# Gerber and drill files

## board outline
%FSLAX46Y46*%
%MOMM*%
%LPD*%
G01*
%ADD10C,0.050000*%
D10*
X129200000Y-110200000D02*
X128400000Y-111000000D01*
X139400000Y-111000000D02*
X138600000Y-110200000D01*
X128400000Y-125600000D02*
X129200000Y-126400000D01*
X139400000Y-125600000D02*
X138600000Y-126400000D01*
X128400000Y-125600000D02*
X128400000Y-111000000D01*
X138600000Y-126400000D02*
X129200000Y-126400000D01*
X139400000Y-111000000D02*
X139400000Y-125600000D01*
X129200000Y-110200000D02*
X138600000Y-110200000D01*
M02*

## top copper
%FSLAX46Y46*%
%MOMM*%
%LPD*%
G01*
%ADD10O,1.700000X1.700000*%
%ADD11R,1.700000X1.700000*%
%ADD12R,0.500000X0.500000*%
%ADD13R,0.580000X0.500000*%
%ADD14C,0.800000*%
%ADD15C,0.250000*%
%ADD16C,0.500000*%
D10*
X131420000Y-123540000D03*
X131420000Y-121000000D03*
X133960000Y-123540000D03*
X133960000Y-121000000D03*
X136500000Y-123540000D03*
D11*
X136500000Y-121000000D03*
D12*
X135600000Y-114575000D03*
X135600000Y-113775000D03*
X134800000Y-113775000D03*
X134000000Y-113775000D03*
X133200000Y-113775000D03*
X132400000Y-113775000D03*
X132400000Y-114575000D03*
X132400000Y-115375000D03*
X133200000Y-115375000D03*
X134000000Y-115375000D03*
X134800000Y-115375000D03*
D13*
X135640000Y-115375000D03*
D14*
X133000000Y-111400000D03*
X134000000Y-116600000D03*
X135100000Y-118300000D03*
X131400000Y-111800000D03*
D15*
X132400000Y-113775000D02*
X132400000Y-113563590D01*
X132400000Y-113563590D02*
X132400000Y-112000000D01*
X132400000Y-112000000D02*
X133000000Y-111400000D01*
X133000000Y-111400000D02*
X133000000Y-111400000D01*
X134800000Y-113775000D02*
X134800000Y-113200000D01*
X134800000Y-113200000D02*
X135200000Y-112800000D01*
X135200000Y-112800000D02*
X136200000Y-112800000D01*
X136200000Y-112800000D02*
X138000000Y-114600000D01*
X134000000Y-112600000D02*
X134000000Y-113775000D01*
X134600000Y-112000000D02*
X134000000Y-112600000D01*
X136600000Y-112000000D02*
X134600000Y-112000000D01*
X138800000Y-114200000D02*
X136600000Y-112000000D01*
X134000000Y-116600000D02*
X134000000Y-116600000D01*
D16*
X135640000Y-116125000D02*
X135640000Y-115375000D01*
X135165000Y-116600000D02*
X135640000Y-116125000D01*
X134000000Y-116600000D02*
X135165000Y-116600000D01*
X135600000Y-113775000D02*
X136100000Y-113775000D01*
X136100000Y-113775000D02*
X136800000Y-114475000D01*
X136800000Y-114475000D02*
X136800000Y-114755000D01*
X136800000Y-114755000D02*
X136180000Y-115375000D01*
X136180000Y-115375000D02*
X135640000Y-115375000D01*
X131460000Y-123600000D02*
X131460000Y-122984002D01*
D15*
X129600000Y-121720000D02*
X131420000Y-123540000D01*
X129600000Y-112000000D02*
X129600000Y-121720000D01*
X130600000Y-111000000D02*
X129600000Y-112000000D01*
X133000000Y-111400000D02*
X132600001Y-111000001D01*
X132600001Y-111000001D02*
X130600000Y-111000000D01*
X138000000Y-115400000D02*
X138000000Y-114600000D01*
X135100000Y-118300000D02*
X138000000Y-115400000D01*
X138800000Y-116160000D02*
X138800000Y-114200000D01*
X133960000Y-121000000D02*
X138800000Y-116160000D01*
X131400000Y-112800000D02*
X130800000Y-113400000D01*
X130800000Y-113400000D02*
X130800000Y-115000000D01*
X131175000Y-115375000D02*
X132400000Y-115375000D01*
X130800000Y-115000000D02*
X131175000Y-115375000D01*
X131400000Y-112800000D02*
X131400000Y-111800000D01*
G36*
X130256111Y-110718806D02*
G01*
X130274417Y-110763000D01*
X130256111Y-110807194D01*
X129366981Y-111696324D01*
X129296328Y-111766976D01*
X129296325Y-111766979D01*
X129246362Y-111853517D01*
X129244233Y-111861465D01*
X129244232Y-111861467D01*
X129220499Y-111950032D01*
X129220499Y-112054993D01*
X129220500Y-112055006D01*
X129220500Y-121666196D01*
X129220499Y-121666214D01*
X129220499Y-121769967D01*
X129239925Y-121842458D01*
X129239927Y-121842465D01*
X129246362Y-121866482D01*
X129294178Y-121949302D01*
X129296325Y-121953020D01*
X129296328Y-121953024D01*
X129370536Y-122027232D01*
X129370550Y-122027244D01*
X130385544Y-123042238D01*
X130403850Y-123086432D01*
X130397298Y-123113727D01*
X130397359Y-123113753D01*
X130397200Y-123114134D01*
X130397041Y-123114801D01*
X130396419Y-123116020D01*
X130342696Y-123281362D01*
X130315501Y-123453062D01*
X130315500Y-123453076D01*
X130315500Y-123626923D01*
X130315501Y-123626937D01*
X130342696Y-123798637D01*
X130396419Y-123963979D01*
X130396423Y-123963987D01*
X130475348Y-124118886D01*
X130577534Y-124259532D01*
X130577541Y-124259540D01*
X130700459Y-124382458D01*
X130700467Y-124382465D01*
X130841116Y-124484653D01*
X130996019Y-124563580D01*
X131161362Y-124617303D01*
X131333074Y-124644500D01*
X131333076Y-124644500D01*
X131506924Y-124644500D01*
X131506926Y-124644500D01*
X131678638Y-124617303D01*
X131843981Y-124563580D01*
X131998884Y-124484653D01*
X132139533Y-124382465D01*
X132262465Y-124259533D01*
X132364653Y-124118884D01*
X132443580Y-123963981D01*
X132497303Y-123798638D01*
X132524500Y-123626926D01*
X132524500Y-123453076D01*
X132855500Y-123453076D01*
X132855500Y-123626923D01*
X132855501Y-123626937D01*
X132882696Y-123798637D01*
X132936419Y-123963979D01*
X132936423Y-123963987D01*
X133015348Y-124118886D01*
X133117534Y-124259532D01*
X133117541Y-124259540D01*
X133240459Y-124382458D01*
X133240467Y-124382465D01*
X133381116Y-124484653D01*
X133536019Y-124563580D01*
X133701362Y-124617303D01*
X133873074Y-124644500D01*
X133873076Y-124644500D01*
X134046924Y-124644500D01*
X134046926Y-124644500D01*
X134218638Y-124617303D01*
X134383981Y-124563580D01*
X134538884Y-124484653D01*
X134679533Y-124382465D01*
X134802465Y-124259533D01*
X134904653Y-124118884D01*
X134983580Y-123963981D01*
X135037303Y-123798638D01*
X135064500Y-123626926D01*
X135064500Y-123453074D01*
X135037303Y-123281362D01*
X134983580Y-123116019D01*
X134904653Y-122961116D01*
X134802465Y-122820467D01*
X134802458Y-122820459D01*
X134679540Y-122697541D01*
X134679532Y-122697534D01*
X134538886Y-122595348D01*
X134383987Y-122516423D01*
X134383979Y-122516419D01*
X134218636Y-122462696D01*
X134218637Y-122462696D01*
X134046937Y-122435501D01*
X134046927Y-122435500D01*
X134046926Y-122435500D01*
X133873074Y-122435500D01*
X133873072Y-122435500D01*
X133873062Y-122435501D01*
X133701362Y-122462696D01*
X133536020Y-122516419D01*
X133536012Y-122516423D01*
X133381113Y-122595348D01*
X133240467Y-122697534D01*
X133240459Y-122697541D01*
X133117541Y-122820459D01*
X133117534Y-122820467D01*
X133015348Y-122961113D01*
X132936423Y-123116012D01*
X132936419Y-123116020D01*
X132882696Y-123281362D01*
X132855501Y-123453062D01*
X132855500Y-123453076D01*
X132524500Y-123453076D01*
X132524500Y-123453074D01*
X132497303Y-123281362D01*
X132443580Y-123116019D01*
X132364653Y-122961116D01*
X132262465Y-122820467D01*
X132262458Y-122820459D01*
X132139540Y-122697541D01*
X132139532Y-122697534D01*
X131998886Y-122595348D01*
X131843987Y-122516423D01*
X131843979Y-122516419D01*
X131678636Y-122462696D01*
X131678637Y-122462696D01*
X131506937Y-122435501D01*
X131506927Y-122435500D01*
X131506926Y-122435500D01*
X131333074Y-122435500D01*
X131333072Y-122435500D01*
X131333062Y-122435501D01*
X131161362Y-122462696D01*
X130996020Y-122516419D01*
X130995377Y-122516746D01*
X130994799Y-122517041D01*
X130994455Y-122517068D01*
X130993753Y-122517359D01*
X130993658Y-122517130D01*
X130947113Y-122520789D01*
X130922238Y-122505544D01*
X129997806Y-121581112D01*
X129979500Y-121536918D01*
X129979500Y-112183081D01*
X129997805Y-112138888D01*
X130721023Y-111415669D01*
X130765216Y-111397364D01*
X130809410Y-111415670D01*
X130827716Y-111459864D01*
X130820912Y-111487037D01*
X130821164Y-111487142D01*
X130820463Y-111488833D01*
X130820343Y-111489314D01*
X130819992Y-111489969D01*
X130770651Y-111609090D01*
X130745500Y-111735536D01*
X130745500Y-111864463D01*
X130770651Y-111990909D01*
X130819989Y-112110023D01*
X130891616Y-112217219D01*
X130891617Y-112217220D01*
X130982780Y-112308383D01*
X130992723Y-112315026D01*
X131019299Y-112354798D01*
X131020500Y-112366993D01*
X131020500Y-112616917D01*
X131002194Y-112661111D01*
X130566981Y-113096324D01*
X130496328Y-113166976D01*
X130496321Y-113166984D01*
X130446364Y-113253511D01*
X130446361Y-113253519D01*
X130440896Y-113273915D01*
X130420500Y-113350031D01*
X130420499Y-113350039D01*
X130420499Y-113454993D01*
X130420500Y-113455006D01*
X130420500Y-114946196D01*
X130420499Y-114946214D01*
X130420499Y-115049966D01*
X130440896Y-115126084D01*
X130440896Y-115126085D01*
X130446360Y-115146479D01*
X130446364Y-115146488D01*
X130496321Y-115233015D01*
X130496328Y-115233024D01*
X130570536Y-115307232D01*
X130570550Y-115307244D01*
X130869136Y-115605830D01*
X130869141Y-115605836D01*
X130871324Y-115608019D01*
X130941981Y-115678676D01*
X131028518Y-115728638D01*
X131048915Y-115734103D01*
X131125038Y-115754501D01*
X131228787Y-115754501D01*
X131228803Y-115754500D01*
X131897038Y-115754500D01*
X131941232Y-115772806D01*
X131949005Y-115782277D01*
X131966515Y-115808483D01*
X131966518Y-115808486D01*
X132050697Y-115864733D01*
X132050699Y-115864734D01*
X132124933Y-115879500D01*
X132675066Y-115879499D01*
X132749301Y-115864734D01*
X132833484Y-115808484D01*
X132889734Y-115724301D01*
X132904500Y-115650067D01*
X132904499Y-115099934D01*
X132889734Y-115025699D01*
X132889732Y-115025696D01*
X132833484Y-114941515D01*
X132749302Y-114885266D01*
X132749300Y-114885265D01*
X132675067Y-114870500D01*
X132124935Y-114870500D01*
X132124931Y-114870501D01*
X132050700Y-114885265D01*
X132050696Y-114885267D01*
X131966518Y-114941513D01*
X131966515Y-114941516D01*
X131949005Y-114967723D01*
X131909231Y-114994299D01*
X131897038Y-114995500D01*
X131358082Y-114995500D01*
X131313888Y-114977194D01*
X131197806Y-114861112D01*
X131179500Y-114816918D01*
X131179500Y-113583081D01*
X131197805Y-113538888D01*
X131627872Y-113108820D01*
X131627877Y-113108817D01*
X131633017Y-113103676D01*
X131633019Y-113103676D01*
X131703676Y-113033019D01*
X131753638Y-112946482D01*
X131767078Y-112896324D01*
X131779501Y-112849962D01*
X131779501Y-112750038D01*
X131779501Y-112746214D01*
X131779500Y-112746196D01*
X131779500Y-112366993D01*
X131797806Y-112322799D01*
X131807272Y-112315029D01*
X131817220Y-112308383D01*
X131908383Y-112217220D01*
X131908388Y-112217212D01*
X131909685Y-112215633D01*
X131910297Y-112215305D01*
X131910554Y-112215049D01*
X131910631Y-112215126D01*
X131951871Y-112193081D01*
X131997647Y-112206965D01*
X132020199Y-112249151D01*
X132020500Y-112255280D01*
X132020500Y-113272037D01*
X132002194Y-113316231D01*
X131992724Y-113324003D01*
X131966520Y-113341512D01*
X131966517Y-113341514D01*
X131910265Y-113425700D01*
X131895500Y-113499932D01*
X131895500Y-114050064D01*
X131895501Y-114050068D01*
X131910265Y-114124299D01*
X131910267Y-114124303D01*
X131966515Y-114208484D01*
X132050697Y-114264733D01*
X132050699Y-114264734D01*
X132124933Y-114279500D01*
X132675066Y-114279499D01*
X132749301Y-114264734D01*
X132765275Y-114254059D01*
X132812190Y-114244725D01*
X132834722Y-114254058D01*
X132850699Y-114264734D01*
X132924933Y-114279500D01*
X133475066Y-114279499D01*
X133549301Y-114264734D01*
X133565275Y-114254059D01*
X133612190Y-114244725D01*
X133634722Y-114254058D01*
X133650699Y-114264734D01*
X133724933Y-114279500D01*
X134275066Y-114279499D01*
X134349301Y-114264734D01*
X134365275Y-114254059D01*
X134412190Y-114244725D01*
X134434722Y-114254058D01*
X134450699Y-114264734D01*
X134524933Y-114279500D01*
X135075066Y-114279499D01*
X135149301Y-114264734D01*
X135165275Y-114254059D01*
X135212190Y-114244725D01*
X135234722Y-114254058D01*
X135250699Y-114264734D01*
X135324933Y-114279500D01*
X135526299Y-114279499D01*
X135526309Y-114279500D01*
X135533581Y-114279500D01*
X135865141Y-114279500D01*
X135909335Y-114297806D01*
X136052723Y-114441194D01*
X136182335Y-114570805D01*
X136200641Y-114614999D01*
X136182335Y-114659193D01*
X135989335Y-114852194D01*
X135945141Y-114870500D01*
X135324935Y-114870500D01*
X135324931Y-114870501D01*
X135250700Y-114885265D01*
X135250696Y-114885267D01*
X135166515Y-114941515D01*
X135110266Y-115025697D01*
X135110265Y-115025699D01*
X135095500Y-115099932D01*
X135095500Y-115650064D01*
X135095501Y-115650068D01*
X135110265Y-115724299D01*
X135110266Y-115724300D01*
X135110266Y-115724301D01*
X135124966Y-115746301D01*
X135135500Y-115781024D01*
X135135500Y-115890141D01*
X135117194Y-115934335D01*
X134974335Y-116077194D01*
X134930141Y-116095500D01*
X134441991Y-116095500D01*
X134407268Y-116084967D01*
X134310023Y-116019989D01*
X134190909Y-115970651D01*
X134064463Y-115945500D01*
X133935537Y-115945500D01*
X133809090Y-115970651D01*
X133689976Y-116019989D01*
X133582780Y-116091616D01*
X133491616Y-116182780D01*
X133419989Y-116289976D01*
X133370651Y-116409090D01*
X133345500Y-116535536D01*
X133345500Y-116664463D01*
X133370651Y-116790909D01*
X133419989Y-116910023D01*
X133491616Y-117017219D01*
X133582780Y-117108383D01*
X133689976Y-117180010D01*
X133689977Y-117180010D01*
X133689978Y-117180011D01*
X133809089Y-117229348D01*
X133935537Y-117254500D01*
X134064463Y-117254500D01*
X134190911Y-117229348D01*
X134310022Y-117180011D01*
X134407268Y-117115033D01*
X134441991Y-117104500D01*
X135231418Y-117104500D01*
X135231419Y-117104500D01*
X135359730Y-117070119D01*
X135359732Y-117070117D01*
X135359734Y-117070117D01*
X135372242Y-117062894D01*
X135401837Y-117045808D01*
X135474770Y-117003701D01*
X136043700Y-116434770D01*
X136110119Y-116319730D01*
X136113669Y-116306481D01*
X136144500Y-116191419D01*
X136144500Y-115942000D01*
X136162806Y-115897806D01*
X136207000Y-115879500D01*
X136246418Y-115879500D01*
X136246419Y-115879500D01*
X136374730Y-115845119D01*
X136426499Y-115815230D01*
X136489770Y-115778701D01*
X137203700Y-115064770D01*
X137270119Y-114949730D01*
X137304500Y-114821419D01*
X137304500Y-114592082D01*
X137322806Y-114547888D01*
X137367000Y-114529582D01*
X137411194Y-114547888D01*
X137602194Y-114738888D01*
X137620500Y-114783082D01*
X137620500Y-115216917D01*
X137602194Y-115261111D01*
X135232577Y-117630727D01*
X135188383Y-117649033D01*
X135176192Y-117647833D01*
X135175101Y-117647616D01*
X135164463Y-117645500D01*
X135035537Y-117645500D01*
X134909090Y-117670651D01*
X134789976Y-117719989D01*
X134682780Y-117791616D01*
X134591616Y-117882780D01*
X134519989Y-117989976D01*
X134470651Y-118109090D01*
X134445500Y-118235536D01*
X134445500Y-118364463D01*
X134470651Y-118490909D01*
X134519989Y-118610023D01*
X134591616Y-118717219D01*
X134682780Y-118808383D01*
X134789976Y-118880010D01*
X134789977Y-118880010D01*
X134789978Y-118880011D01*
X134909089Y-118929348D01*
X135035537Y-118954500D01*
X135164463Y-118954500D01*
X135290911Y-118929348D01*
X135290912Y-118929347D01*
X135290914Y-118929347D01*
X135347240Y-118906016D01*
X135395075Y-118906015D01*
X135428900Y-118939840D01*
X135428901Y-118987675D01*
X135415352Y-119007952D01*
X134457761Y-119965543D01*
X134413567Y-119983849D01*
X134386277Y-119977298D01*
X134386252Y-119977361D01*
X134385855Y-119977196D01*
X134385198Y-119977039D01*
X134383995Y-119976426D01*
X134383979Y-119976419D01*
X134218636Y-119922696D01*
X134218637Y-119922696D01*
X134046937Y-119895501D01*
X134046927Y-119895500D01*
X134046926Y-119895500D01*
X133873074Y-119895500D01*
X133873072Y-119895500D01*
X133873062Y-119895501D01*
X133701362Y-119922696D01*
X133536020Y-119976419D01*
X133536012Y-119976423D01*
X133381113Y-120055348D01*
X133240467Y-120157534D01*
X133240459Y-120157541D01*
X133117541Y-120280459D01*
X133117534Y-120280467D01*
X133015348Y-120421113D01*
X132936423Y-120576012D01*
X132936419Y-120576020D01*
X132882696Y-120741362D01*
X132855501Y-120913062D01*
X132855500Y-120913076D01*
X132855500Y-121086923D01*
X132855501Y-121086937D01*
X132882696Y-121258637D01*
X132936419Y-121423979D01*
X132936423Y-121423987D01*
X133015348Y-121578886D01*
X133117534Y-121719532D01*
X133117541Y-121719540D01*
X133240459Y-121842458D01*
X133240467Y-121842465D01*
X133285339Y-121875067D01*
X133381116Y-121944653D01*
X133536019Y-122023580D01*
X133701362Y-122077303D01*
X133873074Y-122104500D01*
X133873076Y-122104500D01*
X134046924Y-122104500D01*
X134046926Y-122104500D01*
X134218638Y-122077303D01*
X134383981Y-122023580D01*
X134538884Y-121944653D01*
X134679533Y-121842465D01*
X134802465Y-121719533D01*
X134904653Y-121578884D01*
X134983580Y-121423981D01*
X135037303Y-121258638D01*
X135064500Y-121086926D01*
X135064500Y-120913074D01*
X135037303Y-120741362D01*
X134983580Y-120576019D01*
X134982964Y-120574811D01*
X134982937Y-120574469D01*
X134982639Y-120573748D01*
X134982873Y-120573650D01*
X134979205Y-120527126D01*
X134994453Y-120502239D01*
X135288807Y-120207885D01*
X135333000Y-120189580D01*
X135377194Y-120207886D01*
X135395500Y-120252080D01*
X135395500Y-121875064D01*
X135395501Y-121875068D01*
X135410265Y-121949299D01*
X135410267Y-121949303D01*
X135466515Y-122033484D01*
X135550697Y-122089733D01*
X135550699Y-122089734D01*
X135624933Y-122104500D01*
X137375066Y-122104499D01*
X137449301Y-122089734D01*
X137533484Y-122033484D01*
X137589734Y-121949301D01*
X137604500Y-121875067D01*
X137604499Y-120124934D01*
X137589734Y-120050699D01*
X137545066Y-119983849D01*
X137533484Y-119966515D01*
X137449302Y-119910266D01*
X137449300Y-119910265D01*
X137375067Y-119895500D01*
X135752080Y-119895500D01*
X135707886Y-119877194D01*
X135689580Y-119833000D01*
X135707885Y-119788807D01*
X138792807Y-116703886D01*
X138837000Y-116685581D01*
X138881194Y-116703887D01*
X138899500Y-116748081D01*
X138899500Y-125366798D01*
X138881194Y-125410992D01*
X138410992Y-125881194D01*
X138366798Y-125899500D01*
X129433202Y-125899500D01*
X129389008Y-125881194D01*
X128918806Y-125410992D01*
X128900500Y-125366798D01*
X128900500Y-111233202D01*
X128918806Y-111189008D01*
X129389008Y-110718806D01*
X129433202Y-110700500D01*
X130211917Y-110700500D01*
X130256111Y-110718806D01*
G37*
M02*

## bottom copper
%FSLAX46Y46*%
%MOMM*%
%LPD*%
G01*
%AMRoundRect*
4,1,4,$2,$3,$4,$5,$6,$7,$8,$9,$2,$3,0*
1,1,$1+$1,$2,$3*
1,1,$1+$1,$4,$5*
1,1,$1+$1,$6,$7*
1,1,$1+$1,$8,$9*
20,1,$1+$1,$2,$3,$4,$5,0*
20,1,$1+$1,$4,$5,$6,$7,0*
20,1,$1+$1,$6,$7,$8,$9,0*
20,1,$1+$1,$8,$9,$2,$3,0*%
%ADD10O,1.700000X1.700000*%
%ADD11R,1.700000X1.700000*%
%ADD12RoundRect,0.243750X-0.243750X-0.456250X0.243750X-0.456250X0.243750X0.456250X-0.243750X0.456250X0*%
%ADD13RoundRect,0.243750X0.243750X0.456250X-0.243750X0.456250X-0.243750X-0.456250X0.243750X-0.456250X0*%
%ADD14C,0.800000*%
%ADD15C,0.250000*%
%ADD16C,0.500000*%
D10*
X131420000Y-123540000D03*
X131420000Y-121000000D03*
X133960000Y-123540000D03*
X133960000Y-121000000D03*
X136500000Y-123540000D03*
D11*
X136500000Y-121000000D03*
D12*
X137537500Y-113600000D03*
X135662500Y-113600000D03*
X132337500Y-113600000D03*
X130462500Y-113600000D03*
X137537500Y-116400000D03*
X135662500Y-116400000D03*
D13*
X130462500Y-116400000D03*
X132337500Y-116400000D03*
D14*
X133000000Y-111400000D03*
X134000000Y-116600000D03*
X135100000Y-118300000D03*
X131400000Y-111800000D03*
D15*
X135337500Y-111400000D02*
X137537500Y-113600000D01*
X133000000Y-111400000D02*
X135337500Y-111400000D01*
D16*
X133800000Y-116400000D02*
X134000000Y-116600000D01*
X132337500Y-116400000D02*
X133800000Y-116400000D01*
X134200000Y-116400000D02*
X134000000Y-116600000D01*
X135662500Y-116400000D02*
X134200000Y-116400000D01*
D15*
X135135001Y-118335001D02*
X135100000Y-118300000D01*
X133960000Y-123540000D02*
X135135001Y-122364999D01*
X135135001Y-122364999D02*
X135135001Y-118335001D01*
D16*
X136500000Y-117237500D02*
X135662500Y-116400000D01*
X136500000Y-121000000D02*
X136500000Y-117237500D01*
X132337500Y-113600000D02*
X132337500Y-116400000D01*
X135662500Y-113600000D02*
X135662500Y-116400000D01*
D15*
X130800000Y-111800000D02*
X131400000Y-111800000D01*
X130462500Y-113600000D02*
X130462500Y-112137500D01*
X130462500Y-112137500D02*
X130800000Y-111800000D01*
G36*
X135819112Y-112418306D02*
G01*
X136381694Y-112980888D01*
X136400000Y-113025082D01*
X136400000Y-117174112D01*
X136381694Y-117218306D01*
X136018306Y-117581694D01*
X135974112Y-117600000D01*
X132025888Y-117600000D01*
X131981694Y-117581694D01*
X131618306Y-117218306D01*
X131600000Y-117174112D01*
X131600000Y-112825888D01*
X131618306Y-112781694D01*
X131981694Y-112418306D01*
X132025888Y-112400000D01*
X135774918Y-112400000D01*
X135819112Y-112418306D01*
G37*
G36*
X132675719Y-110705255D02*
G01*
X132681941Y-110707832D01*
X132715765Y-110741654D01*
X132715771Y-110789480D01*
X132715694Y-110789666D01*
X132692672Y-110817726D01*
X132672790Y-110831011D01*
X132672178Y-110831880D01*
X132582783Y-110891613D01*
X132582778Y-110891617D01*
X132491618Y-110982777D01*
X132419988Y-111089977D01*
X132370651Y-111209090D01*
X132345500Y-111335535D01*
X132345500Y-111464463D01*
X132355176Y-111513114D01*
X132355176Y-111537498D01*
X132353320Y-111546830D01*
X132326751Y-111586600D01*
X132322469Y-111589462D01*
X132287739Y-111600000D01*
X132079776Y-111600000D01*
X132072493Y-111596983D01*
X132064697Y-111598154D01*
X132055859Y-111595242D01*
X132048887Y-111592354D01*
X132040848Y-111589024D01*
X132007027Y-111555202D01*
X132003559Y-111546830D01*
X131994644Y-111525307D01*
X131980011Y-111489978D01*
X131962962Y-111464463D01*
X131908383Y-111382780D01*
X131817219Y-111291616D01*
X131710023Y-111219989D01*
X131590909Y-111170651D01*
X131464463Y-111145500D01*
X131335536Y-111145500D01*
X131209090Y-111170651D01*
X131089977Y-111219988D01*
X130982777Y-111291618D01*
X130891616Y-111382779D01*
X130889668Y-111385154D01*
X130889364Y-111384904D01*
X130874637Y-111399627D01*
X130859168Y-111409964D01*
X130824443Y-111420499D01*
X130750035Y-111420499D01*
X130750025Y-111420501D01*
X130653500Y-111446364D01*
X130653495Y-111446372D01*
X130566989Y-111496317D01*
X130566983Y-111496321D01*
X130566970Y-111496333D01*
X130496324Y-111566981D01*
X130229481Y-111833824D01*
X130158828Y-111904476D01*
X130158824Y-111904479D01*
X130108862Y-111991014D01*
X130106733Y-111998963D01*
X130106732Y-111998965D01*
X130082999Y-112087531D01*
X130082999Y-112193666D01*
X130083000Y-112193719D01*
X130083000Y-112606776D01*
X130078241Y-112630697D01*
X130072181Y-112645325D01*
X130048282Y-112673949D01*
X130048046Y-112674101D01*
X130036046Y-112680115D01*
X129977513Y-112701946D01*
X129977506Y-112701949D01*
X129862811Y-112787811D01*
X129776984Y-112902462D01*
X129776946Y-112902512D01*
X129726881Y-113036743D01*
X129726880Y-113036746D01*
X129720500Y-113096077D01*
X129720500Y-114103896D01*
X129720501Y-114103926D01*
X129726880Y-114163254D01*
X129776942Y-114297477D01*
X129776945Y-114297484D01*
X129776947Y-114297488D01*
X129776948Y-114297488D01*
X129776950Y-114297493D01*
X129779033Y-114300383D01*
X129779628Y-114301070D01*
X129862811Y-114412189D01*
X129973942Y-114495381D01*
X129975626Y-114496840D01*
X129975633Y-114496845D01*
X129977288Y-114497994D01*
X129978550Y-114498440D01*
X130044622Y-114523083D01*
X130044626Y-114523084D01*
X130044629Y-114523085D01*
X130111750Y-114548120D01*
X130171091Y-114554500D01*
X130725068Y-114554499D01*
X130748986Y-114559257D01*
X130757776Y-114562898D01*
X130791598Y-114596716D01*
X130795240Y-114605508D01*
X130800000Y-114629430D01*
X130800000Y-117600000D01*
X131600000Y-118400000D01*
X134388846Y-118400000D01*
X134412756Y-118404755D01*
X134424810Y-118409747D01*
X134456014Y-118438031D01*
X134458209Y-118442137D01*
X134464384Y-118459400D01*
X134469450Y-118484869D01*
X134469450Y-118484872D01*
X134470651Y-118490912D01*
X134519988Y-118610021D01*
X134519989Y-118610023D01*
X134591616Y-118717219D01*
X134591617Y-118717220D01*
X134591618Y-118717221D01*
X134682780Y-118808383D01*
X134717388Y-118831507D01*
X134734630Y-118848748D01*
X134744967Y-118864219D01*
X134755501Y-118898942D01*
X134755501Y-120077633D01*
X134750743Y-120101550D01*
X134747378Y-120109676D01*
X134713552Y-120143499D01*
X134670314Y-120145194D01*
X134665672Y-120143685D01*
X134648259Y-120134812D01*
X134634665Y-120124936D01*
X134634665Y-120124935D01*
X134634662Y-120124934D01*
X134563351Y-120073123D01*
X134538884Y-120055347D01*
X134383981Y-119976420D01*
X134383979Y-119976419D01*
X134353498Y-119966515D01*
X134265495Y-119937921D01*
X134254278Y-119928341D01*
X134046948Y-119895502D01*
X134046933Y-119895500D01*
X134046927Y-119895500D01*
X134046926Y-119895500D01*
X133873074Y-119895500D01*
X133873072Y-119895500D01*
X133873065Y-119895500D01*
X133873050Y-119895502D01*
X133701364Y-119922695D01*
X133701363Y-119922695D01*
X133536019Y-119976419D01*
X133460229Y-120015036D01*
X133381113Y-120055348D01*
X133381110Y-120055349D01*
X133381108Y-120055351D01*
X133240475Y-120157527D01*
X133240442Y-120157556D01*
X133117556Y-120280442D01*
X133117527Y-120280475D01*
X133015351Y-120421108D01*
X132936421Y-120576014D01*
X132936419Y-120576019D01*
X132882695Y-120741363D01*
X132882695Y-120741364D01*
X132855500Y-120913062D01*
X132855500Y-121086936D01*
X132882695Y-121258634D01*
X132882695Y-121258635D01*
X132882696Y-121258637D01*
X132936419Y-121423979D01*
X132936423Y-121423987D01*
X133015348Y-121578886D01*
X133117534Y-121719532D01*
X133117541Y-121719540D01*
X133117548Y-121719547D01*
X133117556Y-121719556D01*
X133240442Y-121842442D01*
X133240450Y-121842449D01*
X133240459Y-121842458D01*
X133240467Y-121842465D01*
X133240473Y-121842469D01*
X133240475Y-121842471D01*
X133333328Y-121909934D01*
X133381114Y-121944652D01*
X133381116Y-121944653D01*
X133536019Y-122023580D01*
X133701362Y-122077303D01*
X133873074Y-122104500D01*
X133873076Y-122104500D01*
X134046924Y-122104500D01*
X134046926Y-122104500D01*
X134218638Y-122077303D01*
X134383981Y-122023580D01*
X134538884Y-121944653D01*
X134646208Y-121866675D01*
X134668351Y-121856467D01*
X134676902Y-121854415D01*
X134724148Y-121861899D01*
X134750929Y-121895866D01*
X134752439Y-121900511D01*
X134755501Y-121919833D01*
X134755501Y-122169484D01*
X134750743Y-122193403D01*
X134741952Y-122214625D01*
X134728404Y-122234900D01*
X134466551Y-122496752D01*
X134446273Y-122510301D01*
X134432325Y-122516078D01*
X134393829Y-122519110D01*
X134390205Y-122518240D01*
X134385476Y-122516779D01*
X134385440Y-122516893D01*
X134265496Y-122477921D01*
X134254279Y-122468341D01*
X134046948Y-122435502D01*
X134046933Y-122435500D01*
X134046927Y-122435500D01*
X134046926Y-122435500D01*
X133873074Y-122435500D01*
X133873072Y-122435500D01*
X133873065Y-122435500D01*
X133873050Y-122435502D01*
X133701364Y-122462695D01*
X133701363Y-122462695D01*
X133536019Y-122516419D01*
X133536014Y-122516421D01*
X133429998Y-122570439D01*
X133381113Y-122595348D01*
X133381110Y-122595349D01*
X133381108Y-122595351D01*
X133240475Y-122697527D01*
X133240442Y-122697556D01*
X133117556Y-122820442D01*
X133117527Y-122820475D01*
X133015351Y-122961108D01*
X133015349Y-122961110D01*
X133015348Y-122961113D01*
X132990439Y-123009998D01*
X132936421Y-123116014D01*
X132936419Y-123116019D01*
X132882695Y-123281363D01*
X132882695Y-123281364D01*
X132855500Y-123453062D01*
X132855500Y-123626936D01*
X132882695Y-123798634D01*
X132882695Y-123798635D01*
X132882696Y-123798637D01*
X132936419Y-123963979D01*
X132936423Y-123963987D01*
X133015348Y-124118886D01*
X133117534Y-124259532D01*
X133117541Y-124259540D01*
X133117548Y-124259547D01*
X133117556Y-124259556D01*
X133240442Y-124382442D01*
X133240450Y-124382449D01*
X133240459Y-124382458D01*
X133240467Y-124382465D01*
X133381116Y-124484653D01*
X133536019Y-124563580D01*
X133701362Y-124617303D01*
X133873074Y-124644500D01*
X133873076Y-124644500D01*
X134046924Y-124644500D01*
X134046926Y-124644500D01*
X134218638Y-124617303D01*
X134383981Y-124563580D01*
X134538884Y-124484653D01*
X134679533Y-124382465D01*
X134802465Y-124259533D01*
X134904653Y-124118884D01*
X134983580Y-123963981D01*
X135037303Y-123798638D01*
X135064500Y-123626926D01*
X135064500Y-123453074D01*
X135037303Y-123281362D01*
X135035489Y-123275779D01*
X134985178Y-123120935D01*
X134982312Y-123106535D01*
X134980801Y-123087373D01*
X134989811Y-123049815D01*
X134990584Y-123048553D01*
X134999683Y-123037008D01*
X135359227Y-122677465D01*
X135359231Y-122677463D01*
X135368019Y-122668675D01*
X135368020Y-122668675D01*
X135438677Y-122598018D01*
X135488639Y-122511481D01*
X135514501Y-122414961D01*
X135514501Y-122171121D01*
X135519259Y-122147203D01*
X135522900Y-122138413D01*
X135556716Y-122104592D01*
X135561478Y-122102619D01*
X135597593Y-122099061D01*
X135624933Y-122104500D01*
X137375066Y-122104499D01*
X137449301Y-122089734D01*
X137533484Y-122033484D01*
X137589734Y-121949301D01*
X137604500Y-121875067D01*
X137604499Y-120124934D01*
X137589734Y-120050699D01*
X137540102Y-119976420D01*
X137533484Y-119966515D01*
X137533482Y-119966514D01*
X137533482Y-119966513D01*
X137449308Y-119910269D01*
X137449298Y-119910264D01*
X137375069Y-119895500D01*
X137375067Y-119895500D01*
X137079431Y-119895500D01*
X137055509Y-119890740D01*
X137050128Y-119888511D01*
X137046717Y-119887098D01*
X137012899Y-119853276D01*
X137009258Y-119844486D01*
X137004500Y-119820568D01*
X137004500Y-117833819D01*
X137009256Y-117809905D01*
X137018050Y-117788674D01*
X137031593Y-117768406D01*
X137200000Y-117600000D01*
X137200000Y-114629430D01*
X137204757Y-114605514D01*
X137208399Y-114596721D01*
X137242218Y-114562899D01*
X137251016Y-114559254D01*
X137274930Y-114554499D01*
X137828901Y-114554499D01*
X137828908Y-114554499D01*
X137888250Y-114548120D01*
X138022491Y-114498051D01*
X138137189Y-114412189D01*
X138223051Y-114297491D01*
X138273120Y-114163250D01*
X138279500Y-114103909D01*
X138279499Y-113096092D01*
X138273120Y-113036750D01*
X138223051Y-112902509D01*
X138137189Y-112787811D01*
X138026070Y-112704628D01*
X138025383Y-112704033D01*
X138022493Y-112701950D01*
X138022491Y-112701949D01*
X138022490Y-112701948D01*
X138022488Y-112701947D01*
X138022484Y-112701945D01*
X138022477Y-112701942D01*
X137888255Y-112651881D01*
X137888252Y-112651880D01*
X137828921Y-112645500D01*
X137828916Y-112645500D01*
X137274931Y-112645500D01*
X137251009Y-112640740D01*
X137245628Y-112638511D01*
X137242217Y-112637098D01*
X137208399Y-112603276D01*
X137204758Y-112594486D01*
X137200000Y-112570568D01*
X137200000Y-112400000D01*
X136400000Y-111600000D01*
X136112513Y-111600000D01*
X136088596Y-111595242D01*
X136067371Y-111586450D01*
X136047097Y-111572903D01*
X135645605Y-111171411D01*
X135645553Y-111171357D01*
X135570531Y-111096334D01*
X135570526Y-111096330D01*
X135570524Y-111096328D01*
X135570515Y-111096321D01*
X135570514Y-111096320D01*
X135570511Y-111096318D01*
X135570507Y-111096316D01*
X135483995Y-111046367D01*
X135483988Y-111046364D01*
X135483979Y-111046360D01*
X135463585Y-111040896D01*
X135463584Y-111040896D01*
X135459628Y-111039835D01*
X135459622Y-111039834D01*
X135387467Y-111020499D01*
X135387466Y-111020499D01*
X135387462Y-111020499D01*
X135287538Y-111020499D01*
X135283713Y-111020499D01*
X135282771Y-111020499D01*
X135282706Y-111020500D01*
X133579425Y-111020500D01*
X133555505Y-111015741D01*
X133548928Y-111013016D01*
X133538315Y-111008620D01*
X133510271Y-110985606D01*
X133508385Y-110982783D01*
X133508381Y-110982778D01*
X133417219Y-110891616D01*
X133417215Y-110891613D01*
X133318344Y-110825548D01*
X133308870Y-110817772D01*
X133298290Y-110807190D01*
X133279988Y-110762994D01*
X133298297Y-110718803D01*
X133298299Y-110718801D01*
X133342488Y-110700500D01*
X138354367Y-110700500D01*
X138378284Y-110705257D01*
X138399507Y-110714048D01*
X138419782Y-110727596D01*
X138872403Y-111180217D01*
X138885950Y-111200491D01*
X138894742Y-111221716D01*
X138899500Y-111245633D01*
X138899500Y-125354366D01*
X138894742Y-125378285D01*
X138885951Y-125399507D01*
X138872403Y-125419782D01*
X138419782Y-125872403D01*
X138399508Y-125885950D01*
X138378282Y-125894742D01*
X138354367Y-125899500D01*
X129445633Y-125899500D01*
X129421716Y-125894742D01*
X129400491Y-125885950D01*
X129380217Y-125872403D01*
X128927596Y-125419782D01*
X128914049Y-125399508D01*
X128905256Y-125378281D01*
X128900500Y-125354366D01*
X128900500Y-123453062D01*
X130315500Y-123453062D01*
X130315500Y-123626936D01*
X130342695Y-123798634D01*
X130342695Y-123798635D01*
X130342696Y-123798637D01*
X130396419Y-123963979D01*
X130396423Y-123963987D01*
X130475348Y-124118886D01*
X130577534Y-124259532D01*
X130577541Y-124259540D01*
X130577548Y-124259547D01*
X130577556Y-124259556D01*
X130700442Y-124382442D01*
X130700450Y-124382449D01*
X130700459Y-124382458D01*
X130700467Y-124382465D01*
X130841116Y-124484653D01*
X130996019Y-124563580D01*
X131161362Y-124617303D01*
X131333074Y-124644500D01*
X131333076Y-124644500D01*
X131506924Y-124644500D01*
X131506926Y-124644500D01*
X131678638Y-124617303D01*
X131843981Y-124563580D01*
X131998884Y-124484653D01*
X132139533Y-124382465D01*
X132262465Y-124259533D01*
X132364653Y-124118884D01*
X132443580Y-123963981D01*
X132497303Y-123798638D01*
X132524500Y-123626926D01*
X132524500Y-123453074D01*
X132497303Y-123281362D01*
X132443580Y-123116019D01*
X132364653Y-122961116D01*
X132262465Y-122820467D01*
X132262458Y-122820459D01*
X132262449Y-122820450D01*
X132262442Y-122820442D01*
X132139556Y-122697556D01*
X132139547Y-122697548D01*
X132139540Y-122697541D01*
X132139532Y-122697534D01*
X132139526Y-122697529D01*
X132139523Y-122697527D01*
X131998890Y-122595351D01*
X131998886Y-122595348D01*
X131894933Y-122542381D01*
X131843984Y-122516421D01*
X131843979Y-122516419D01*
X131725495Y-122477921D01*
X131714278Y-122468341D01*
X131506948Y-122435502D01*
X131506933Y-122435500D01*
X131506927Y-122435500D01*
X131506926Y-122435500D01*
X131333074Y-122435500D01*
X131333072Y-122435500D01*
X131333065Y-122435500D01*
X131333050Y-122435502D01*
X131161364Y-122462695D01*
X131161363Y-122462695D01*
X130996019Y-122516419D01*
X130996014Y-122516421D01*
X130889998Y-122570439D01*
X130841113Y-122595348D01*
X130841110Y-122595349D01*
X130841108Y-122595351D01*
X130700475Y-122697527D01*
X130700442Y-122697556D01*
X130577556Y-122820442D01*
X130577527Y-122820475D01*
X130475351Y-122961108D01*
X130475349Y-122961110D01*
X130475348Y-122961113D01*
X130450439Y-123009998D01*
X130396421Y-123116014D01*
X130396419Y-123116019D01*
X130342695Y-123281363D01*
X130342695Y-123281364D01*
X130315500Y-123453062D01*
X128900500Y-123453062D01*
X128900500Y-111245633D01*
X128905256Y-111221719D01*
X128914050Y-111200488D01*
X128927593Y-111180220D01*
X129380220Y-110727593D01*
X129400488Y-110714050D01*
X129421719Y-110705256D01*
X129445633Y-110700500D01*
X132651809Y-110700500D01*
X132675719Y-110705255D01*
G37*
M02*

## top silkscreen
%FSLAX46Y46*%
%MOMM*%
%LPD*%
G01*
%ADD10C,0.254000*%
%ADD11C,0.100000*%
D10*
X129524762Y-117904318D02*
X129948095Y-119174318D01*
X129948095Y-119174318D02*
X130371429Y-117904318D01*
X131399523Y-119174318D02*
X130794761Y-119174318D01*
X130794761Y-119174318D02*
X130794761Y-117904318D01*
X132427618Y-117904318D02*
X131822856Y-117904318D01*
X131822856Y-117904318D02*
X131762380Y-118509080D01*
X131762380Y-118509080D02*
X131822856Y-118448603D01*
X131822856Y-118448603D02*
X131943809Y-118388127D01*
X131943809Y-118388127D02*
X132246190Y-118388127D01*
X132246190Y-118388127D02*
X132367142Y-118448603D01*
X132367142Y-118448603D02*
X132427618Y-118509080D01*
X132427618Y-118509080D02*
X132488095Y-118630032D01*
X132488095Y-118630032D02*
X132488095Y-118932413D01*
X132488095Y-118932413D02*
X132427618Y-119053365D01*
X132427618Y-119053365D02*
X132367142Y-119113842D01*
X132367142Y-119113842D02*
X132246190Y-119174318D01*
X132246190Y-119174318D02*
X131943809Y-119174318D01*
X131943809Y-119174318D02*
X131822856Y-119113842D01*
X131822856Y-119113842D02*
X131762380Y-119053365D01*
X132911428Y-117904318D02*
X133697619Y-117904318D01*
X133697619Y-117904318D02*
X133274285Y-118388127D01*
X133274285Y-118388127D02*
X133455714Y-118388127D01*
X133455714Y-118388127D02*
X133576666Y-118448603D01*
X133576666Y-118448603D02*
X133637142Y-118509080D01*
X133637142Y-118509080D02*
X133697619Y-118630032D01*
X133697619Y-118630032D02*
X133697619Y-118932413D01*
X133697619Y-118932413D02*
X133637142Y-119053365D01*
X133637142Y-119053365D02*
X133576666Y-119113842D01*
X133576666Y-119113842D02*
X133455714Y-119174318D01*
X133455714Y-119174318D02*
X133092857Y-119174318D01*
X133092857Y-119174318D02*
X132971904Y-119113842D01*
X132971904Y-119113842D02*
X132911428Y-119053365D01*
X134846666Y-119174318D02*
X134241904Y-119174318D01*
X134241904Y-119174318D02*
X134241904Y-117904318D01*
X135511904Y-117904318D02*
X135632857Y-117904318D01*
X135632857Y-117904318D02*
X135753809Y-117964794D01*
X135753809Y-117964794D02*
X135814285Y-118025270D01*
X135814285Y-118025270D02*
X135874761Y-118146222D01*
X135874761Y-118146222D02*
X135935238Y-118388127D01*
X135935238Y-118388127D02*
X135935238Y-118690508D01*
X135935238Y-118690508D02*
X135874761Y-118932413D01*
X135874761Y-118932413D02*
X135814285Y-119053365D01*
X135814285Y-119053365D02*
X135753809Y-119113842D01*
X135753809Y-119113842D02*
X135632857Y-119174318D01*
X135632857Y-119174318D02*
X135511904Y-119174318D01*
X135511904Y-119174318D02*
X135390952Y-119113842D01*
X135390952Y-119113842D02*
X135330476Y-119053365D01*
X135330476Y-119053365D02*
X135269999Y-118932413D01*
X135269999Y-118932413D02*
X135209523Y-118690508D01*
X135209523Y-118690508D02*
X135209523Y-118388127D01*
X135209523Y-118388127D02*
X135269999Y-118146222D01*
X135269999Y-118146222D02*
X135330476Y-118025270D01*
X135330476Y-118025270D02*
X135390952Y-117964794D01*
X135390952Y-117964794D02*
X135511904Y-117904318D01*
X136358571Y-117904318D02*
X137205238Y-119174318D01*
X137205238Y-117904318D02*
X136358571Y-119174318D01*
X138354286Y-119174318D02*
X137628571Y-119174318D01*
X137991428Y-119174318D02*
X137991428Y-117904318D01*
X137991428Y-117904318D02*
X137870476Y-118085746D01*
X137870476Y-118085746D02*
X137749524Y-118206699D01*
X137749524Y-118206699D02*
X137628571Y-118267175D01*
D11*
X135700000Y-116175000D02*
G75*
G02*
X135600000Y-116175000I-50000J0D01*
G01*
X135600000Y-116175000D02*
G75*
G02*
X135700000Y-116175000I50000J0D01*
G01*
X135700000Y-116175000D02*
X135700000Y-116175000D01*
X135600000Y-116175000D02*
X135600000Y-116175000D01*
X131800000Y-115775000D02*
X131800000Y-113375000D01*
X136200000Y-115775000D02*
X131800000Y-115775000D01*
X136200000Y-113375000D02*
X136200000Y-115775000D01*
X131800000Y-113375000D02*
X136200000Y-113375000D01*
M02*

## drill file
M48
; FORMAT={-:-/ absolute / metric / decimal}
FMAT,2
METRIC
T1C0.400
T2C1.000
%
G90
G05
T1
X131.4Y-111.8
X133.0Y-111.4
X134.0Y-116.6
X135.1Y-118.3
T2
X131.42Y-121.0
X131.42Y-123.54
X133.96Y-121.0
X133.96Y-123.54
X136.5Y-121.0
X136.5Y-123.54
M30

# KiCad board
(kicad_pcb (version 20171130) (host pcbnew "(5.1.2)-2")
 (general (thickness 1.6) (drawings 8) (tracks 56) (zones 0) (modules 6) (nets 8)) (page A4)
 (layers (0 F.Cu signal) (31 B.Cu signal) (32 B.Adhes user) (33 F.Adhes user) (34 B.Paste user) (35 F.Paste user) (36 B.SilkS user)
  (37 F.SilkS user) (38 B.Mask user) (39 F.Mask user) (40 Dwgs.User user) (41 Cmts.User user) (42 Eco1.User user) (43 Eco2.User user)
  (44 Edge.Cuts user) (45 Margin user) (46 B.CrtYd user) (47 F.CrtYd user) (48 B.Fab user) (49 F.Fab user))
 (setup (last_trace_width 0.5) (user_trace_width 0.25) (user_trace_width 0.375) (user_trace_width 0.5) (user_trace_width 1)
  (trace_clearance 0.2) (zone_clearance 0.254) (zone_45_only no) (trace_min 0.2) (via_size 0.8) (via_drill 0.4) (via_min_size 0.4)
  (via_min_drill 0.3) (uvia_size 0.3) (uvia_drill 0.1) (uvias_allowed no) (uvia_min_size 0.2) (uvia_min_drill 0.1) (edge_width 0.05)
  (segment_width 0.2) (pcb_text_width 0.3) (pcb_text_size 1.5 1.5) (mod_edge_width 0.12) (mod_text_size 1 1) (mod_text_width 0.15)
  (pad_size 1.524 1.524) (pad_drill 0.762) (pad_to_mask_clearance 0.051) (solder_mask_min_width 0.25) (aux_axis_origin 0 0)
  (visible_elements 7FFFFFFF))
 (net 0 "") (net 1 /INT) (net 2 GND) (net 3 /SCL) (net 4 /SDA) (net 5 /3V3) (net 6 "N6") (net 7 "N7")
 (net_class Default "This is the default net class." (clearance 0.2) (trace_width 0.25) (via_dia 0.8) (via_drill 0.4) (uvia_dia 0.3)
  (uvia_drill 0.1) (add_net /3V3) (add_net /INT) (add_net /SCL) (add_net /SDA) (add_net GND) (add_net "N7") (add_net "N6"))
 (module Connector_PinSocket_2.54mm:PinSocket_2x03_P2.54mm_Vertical (layer B.Cu) (at 136.5 121 90)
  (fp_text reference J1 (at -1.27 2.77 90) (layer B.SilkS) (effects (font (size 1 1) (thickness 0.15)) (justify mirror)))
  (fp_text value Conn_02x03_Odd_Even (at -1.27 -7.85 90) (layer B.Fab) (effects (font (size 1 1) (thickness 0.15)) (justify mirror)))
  (pad 6 thru_hole oval (at -2.54 -5.08 90) (size 1.7 1.7) (drill 1) (layers *.Cu *.Mask) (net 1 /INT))
  (pad 5 thru_hole oval (at 0 -5.08 90) (size 1.7 1.7) (drill 1) (layers *.Cu *.Mask) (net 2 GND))
  (pad 4 thru_hole oval (at -2.54 -2.54 90) (size 1.7 1.7) (drill 1) (layers *.Cu *.Mask) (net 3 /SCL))
  (pad 3 thru_hole oval (at 0 -2.54 90) (size 1.7 1.7) (drill 1) (layers *.Cu *.Mask) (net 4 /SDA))
  (pad 2 thru_hole oval (at -2.54 0 90) (size 1.7 1.7) (drill 1) (layers *.Cu *.Mask) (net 2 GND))
  (pad 1 thru_hole rect (at 0 0 90) (size 1.7 1.7) (drill 1) (layers *.Cu *.Mask) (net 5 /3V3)))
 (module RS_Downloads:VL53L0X (layer F.Cu) (at 134 114.8)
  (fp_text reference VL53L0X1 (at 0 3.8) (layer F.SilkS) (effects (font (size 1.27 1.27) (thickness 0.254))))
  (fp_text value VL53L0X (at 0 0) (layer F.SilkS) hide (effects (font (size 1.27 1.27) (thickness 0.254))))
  (fp_arc (start 1.65 1.375) (end 1.7 1.375) (angle 180) (layer F.SilkS) (width 0.1))
  (fp_arc (start 1.65 1.375) (end 1.6 1.375) (angle 180) (layer F.SilkS) (width 0.1))
  (fp_line (start 1.7 1.375) (end 1.7 1.375) (layer F.SilkS) (width 0.1))
  (fp_line (start 1.6 1.375) (end 1.6 1.375) (layer F.SilkS) (width 0.1))
  (fp_line (start -2.2 0.975) (end -2.2 -1.425) (layer F.SilkS) (width 0.1))
  (fp_line (start 2.2 0.975) (end -2.2 0.975) (layer F.SilkS) (width 0.1))
  (fp_line (start 2.2 -1.425) (end 2.2 0.975) (layer F.SilkS) (width 0.1))
  (fp_line (start -2.2 -1.425) (end 2.2 -1.425) (layer F.SilkS) (width 0.1))
  (pad 12 smd rect (at 1.6 -0.225 90) (size 0.5 0.5) (layers F.Cu F.Paste F.Mask) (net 2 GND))
  (pad 11 smd rect (at 1.6 -1.025 90) (size 0.5 0.5) (layers F.Cu F.Paste F.Mask) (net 5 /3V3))
  (pad 10 smd rect (at 0.8 -1.025 90) (size 0.5 0.5) (layers F.Cu F.Paste F.Mask) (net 3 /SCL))
  (pad 9 smd rect (at 0 -1.025 90) (size 0.5 0.5) (layers F.Cu F.Paste F.Mask) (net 4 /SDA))
  (pad 8 smd rect (at -0.8 -1.025 90) (size 0.5 0.5) (layers F.Cu F.Paste F.Mask) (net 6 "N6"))
  (pad 7 smd rect (at -1.6 -1.025 90) (size 0.5 0.5) (layers F.Cu F.Paste F.Mask) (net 1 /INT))
  (pad 6 smd rect (at -1.6 -0.225 90) (size 0.5 0.5) (layers F.Cu F.Paste F.Mask) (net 2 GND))
  (pad 5 smd rect (at -1.6 0.575 90) (size 0.5 0.5) (layers F.Cu F.Paste F.Mask) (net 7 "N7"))
  (pad 4 smd rect (at -0.8 0.575 90) (size 0.5 0.5) (layers F.Cu F.Paste F.Mask) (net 2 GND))
  (pad 3 smd rect (at 0 0.575 90) (size 0.5 0.5) (layers F.Cu F.Paste F.Mask) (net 2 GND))
  (pad 2 smd rect (at 0.8 0.575 90) (size 0.5 0.5) (layers F.Cu F.Paste F.Mask) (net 2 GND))
  (pad 1 smd rect (at 1.64 0.575 90) (size 0.5 0.58) (layers F.Cu F.Paste F.Mask) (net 5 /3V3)))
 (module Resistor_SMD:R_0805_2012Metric (layer B.Cu) (at 136.6 113.6)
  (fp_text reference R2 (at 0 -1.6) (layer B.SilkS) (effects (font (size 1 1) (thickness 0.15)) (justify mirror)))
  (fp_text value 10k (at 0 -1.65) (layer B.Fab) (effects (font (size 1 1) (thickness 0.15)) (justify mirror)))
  (pad 2 smd roundrect (at 0.9375 0) (size 0.975 1.4) (layers B.Cu B.Paste B.Mask) (roundrect_rratio 0.25) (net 1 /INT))
  (pad 1 smd roundrect (at -0.9375 0) (size 0.975 1.4) (layers B.Cu B.Paste B.Mask) (roundrect_rratio 0.25) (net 5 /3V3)))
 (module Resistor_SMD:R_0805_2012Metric (layer B.Cu) (at 131.4 113.6)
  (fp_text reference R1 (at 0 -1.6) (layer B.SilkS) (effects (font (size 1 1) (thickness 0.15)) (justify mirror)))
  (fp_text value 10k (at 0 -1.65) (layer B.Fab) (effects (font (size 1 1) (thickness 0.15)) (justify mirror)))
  (pad 2 smd roundrect (at 0.9375 0) (size 0.975 1.4) (layers B.Cu B.Paste B.Mask) (roundrect_rratio 0.25) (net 5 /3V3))
  (pad 1 smd roundrect (at -0.9375 0) (size 0.975 1.4) (layers B.Cu B.Paste B.Mask) (roundrect_rratio 0.25) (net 7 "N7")))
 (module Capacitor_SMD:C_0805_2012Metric (layer B.Cu) (at 136.6 116.4)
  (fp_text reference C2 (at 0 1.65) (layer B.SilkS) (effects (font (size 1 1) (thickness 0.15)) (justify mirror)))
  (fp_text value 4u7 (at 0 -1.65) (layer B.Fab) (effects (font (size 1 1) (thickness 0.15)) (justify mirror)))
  (pad 2 smd roundrect (at 0.9375 0) (size 0.975 1.4) (layers B.Cu B.Paste B.Mask) (roundrect_rratio 0.25) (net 2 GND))
  (pad 1 smd roundrect (at -0.9375 0) (size 0.975 1.4) (layers B.Cu B.Paste B.Mask) (roundrect_rratio 0.25) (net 5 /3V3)))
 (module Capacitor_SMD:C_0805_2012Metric (layer B.Cu) (at 131.4 116.4 180)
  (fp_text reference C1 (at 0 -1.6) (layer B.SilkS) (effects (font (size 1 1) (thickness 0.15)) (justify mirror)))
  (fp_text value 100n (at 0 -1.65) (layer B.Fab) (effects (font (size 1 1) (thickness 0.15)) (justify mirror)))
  (pad 2 smd roundrect (at 0.9375 0 180) (size 0.975 1.4) (layers B.Cu B.Paste B.Mask) (roundrect_rratio 0.25) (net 2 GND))
  (pad 1 smd roundrect (at -0.9375 0 180) (size 0.975 1.4) (layers B.Cu B.Paste B.Mask) (roundrect_rratio 0.25) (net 5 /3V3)))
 (gr_line (start 129.2 110.2) (end 128.4 111) (layer Edge.Cuts) (width 0.05))
 (gr_line (start 139.4 111) (end 138.6 110.2) (layer Edge.Cuts) (width 0.05))
 (gr_line (start 128.4 125.6) (end 129.2 126.4) (layer Edge.Cuts) (width 0.05))
 (gr_line (start 139.4 125.6) (end 138.6 126.4) (layer Edge.Cuts) (width 0.05))
 (gr_line (start 128.4 125.6) (end 128.4 111) (layer Edge.Cuts) (width 0.05))
 (gr_line (start 138.6 126.4) (end 129.2 126.4) (layer Edge.Cuts) (width 0.05))
 (gr_line (start 139.4 111) (end 139.4 125.6) (layer Edge.Cuts) (width 0.05))
 (gr_line (start 129.2 110.2) (end 138.6 110.2) (layer Edge.Cuts) (width 0.05))
 (segment (start 132.4 113.775) (end 132.4 113.56359) (width 0.25) (layer F.Cu) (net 1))
 (segment (start 132.4 113.56359) (end 132.4 112) (width 0.25) (layer F.Cu) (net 1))
 (segment (start 132.4 112) (end 133 111.4) (width 0.25) (layer F.Cu) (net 1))
 (segment (start 133 111.4) (end 133 111.4) (width 0.25) (layer F.Cu) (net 1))
 (via (at 133 111.4) (size 0.8) (drill 0.4) (layers F.Cu B.Cu) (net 1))
 (segment (start 135.3375 111.4) (end 137.5375 113.6) (width 0.25) (layer B.Cu) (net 1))
 (segment (start 133 111.4) (end 135.3375 111.4) (width 0.25) (layer B.Cu) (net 1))
 (segment (start 134.8 113.775) (end 134.8 113.2) (width 0.25) (layer F.Cu) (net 3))
 (segment (start 134.8 113.2) (end 135.2 112.8) (width 0.25) (layer F.Cu) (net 3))
 (segment (start 135.2 112.8) (end 136.2 112.8) (width 0.25) (layer F.Cu) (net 3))
 (segment (start 136.2 112.8) (end 138 114.6) (width 0.25) (layer F.Cu) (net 3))
 (segment (start 134 112.6) (end 134 113.775) (width 0.25) (layer F.Cu) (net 4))
 (segment (start 134.6 112) (end 134 112.6) (width 0.25) (layer F.Cu) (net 4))
 (segment (start 136.6 112) (end 134.6 112) (width 0.25) (layer F.Cu) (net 4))
 (segment (start 138.8 114.2) (end 136.6 112) (width 0.25) (layer F.Cu) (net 4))
 (segment (start 134 116.6) (end 134 116.6) (width 0.25) (layer F.Cu) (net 5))
 (via (at 134 116.6) (size 0.8) (drill 0.4) (layers F.Cu B.Cu) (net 5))
 (segment (start 135.64 116.125) (end 135.64 115.375) (width 0.5) (layer F.Cu) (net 5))
 (segment (start 135.165 116.6) (end 135.64 116.125) (width 0.5) (layer F.Cu) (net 5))
 (segment (start 134 116.6) (end 135.165 116.6) (width 0.5) (layer F.Cu) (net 5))
 (segment (start 135.6 113.775) (end 136.1 113.775) (width 0.5) (layer F.Cu) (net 5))
 (segment (start 136.1 113.775) (end 136.8 114.475) (width 0.5) (layer F.Cu) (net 5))
 (segment (start 136.8 114.475) (end 136.8 114.755) (width 0.5) (layer F.Cu) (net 5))
 (segment (start 136.8 114.755) (end 136.18 115.375) (width 0.5) (layer F.Cu) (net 5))
 (segment (start 136.18 115.375) (end 135.64 115.375) (width 0.5) (layer F.Cu) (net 5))
 (segment (start 133.8 116.4) (end 134 116.6) (width 0.5) (layer B.Cu) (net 5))
 (segment (start 132.3375 116.4) (end 133.8 116.4) (width 0.5) (layer B.Cu) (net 5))
 (segment (start 134.2 116.4) (end 134 116.6) (width 0.5) (layer B.Cu) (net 5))
 (segment (start 135.6625 116.4) (end 134.2 116.4) (width 0.5) (layer B.Cu) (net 5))
 (segment (start 131.46 123.6) (end 131.46 122.984002) (width 0.5) (layer F.Cu) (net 1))
 (segment (start 129.6 121.72) (end 131.42 123.54) (width 0.25) (layer F.Cu) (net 1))
 (segment (start 129.6 112) (end 129.6 121.72) (width 0.25) (layer F.Cu) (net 1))
 (segment (start 130.6 111) (end 129.6 112) (width 0.25) (layer F.Cu) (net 1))
 (segment (start 133 111.4) (end 132.600001 111.000001) (width 0.25) (layer F.Cu) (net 1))
 (segment (start 132.600001 111.000001) (end 130.6 111) (width 0.25) (layer F.Cu) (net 1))
 (via (at 135.1 118.3) (size 0.8) (drill 0.4) (layers F.Cu B.Cu) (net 3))
 (segment (start 135.135001 118.335001) (end 135.1 118.3) (width 0.25) (layer B.Cu) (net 3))
 (segment (start 133.96 123.54) (end 135.135001 122.364999) (width 0.25) (layer B.Cu) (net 3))
 (segment (start 135.135001 122.364999) (end 135.135001 118.335001) (width 0.25) (layer B.Cu) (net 3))
 (segment (start 138 115.4) (end 138 114.6) (width 0.25) (layer F.Cu) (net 3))
 (segment (start 135.1 118.3) (end 138 115.4) (width 0.25) (layer F.Cu) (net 3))
 (segment (start 138.8 116.16) (end 138.8 114.2) (width 0.25) (layer F.Cu) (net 4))
 (segment (start 133.96 121) (end 138.8 116.16) (width 0.25) (layer F.Cu) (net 4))
 (segment (start 136.5 117.2375) (end 135.6625 116.4) (width 0.5) (layer B.Cu) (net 5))
 (segment (start 136.5 121) (end 136.5 117.2375) (width 0.5) (layer B.Cu) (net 5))
 (segment (start 132.3375 113.6) (end 132.3375 116.4) (width 0.5) (layer B.Cu) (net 5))
 (segment (start 135.6625 113.6) (end 135.6625 116.4) (width 0.5) (layer B.Cu) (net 5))
 (via (at 131.4 111.8) (size 0.8) (drill 0.4) (layers F.Cu B.Cu) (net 7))
 (segment (start 131.4 112.8) (end 130.8 113.4) (width 0.25) (layer F.Cu) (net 7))
 (segment (start 130.8 113.4) (end 130.8 115) (width 0.25) (layer F.Cu) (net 7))
 (segment (start 131.175 115.375) (end 132.4 115.375) (width 0.25) (layer F.Cu) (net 7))
 (segment (start 130.8 115) (end 131.175 115.375) (width 0.25) (layer F.Cu) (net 7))
 (segment (start 131.4 112.8) (end 131.4 111.8) (width 0.25) (layer F.Cu) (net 7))
 (segment (start 130.8 111.8) (end 131.4 111.8) (width 0.25) (layer B.Cu) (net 7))
 (segment (start 130.4625 113.6) (end 130.4625 112.1375) (width 0.25) (layer B.Cu) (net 7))
 (segment (start 130.4625 112.1375) (end 130.8 111.8) (width 0.25) (layer B.Cu) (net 7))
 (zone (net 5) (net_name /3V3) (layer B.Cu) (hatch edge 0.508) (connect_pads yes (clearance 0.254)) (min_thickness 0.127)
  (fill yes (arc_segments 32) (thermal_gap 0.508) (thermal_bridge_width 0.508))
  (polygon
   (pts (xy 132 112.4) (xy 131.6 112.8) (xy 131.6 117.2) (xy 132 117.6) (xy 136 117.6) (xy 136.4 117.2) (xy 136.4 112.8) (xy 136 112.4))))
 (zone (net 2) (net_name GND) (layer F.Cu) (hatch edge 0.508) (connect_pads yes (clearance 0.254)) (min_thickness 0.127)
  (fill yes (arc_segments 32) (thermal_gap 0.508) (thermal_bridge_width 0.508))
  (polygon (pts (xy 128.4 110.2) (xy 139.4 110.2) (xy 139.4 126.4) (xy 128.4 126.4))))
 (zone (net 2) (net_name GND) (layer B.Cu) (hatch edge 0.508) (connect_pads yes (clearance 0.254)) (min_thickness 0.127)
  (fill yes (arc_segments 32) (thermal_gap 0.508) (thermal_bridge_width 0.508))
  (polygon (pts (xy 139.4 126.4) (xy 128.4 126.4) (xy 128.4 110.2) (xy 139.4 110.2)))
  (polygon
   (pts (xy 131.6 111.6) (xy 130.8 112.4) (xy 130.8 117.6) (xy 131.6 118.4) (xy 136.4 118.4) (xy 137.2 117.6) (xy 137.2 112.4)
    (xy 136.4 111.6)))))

